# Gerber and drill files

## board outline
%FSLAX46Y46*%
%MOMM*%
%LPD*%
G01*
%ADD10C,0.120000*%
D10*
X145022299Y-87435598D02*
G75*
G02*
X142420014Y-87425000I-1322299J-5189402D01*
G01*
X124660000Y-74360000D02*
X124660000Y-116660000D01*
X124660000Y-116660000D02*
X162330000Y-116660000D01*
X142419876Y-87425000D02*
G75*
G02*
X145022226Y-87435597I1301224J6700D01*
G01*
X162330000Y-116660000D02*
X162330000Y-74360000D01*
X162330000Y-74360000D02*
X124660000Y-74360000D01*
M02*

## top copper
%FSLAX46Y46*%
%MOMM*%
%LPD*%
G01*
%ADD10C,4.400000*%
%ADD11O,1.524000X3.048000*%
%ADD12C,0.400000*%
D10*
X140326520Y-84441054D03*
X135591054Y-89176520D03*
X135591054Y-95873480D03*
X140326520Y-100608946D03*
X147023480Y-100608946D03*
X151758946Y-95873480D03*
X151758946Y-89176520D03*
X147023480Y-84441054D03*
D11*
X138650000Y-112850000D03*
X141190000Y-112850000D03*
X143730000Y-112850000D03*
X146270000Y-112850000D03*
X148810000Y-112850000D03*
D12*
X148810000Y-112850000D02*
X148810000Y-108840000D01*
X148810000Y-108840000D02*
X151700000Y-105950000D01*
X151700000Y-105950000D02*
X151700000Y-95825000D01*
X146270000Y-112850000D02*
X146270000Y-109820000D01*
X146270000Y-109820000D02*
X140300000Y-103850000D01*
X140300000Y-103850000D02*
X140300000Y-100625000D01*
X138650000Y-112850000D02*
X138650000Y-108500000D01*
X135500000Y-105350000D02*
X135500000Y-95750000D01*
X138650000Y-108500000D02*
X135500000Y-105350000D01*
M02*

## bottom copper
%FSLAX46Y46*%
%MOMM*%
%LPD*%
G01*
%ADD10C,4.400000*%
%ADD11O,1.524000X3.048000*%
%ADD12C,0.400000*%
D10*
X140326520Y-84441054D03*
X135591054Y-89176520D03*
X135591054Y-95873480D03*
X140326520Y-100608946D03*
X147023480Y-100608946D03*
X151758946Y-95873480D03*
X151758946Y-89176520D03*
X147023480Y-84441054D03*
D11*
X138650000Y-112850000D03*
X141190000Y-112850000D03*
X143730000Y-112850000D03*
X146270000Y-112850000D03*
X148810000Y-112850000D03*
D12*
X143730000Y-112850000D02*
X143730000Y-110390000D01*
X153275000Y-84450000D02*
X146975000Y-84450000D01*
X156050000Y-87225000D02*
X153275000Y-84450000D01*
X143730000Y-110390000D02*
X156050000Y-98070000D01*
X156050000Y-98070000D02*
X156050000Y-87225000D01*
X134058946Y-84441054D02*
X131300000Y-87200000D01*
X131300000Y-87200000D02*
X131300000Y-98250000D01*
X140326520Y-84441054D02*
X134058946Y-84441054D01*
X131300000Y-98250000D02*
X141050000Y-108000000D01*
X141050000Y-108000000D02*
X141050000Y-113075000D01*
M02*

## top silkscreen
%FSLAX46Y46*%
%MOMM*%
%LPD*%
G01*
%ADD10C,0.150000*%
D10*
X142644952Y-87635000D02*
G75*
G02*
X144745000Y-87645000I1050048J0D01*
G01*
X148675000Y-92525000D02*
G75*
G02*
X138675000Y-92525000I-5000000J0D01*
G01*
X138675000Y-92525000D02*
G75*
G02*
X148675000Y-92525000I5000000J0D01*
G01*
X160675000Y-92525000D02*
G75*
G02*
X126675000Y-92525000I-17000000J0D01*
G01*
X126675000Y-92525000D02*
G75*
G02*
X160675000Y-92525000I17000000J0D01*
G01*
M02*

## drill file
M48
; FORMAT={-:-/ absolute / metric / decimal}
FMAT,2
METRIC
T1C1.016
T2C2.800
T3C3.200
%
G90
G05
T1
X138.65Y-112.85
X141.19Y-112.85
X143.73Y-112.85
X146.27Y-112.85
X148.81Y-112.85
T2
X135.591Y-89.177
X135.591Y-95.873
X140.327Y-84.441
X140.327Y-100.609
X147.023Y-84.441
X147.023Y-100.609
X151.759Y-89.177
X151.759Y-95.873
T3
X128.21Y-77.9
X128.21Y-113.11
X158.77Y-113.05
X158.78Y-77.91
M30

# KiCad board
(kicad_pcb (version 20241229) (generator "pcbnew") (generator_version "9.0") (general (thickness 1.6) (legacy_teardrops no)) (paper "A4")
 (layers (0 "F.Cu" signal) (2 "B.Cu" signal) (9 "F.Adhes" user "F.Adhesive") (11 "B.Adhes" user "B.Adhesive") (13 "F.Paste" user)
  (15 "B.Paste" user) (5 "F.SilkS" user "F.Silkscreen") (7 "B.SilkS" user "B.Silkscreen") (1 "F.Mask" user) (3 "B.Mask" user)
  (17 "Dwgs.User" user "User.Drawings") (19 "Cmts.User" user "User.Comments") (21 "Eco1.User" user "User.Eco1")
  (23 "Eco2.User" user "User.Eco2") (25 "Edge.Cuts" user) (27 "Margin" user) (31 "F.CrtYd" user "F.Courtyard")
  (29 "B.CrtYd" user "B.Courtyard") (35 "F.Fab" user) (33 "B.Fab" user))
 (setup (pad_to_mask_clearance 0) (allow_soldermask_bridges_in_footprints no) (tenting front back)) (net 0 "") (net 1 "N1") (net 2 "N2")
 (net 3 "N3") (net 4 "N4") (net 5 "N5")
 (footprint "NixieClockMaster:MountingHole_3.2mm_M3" (layer "F.Cu") (at 128.21 77.9)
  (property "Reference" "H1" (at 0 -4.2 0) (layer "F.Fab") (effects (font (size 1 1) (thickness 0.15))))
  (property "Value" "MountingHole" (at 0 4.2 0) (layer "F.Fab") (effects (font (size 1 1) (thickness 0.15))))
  (pad "" np_thru_hole circle (at 0 0) (size 3.2 3.2) (drill 3.2) (layers "*.Cu" "*.Mask")))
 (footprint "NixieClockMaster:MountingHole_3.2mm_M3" (layer "F.Cu") (at 128.21 113.11)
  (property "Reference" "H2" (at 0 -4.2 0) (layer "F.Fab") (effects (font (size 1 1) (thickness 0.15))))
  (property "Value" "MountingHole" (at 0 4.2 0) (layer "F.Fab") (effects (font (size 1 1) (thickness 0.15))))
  (pad "" np_thru_hole circle (at 0 0) (size 3.2 3.2) (drill 3.2) (layers "*.Cu" "*.Mask")))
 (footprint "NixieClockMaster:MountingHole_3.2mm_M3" (layer "F.Cu") (at 158.78 77.91)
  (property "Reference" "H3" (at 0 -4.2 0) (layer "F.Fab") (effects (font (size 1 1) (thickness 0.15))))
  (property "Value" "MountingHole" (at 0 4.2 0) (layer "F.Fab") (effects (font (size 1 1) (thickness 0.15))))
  (pad "" np_thru_hole circle (at 0 0) (size 3.2 3.2) (drill 3.2) (layers "*.Cu" "*.Mask")))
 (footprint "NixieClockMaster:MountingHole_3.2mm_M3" (layer "F.Cu") (at 158.77 113.05)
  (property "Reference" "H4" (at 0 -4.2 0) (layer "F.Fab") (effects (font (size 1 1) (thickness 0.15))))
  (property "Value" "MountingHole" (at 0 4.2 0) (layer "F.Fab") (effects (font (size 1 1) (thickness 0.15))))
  (pad "" np_thru_hole circle (at 0 0) (size 3.2 3.2) (drill 3.2) (layers "*.Cu" "*.Mask")))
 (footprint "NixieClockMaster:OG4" (layer "F.Cu") (at 143.675 92.525)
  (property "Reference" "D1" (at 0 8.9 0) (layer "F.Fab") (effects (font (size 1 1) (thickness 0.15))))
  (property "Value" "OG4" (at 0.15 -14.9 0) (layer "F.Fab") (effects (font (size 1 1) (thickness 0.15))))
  (fp_arc (start -1.030048 -4.89) (mid 0.025 -5.940036) (end 1.07 -4.88) (stroke (width 0.15) (type solid)) (layer "F.SilkS"))
  (fp_circle (center 0 0) (end 5 0) (stroke (width 0.15) (type solid)) (fill no) (layer "F.SilkS"))
  (fp_circle (center 0 0) (end 17 0) (stroke (width 0.15) (type solid)) (fill no) (layer "F.SilkS"))
  (pad "1" thru_hole circle (at -3.34848 -8.083946) (size 4.4 4.4) (drill 2.8) (layers "*.Cu" "*.Mask") (remove_unused_layers no)
   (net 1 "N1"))
  (pad "2" thru_hole circle (at -8.083946 -3.34848) (size 4.4 4.4) (drill 2.8) (layers "*.Cu" "*.Mask") (remove_unused_layers no))
  (pad "3" thru_hole circle (at -8.083946 3.34848) (size 4.4 4.4) (drill 2.8) (layers "*.Cu" "*.Mask") (remove_unused_layers no)
   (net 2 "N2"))
  (pad "4" thru_hole circle (at -3.34848 8.083946) (size 4.4 4.4) (drill 2.8) (layers "*.Cu" "*.Mask") (remove_unused_layers no)
   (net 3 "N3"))
  (pad "5" thru_hole circle (at 3.34848 8.083946) (size 4.4 4.4) (drill 2.8) (layers "*.Cu" "*.Mask") (remove_unused_layers no))
  (pad "6" thru_hole circle (at 8.083946 3.34848) (size 4.4 4.4) (drill 2.8) (layers "*.Cu" "*.Mask") (remove_unused_layers no) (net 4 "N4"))
  (pad "7" thru_hole circle (at 8.083946 -3.34848) (size 4.4 4.4) (drill 2.8) (layers "*.Cu" "*.Mask") (remove_unused_layers no))
  (pad "8" thru_hole circle (at 3.34848 -8.083946) (size 4.4 4.4) (drill 2.8) (layers "*.Cu" "*.Mask") (remove_unused_layers no)
   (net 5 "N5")))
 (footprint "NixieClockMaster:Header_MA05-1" (layer "B.Cu") (at 145 112.85)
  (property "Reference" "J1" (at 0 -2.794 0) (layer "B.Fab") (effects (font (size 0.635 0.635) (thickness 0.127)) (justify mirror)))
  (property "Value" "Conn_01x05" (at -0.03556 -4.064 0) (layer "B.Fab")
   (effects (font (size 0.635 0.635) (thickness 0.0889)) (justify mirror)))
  (pad "1" thru_hole oval (at -6.35 0 180) (size 1.524 3.048) (drill 1.016) (layers "*.Cu" "*.Mask") (remove_unused_layers no) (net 2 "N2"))
  (pad "2" thru_hole oval (at -3.81 0 180) (size 1.524 3.048) (drill 1.016) (layers "*.Cu" "*.Mask") (remove_unused_layers no) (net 1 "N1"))
  (pad "3" thru_hole oval (at -1.27 0 180) (size 1.524 3.048) (drill 1.016) (layers "*.Cu" "*.Mask") (remove_unused_layers no) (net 5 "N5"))
  (pad "4" thru_hole oval (at 1.27 0 180) (size 1.524 3.048) (drill 1.016) (layers "*.Cu" "*.Mask") (remove_unused_layers no) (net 3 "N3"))
  (pad "5" thru_hole oval (at 3.81 0 180) (size 1.524 3.048) (drill 1.016) (layers "*.Cu" "*.Mask") (remove_unused_layers no) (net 4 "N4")))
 (gr_arc (start 145.022299 87.435598) (mid 143.67819 97.980174) (end 142.420014 87.425) (stroke (width 0.12) (type solid))
  (layer "Edge.Cuts"))
 (gr_line (start 124.66 74.36) (end 124.66 116.66) (stroke (width 0.12) (type solid)) (layer "Edge.Cuts"))
 (gr_line (start 124.66 116.66) (end 162.33 116.66) (stroke (width 0.12) (type solid)) (layer "Edge.Cuts"))
 (gr_arc (start 142.419876 87.425) (mid 143.726435 86.117072) (end 145.022299 87.435598) (stroke (width 0.12) (type solid))
  (layer "Edge.Cuts"))
 (gr_line (start 162.33 116.66) (end 162.33 74.36) (stroke (width 0.12) (type solid)) (layer "Edge.Cuts"))
 (gr_line (start 162.33 74.36) (end 124.66 74.36) (stroke (width 0.12) (type solid)) (layer "Edge.Cuts"))
 (segment (start 143.73 112.85) (end 143.73 110.39) (width 0.4) (layer "B.Cu") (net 5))
 (segment (start 153.275 84.45) (end 146.975 84.45) (width 0.4) (layer "B.Cu") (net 5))
 (segment (start 156.05 87.225) (end 153.275 84.45) (width 0.4) (layer "B.Cu") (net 5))
 (segment (start 143.73 110.39) (end 156.05 98.07) (width 0.4) (layer "B.Cu") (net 5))
 (segment (start 156.05 98.07) (end 156.05 87.225) (width 0.4) (layer "B.Cu") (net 5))
 (segment (start 148.81 112.85) (end 148.81 108.84) (width 0.4) (layer "F.Cu") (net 4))
 (segment (start 148.81 108.84) (end 151.7 105.95) (width 0.4) (layer "F.Cu") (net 4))
 (segment (start 151.7 105.95) (end 151.7 95.825) (width 0.4) (layer "F.Cu") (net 4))
 (segment (start 146.27 112.85) (end 146.27 109.82) (width 0.4) (layer "F.Cu") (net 3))
 (segment (start 146.27 109.82) (end 140.3 103.85) (width 0.4) (layer "F.Cu") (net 3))
 (segment (start 140.3 103.85) (end 140.3 100.625) (width 0.4) (layer "F.Cu") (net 3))
 (segment (start 138.65 112.85) (end 138.65 108.5) (width 0.4) (layer "F.Cu") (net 2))
 (segment (start 135.5 105.35) (end 135.5 95.75) (width 0.4) (layer "F.Cu") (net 2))
 (segment (start 138.65 108.5) (end 135.5 105.35) (width 0.4) (layer "F.Cu") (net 2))
 (segment (start 134.058946 84.441054) (end 131.3 87.2) (width 0.4) (layer "B.Cu") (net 1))
 (segment (start 131.3 87.2) (end 131.3 98.25) (width 0.4) (layer "B.Cu") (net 1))
 (segment (start 140.32652 84.441054) (end 134.058946 84.441054) (width 0.4) (layer "B.Cu") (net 1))
 (segment (start 131.3 98.25) (end 141.05 108) (width 0.4) (layer "B.Cu") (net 1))
 (segment (start 141.05 108) (end 141.05 113.075) (width 0.4) (layer "B.Cu") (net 1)))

